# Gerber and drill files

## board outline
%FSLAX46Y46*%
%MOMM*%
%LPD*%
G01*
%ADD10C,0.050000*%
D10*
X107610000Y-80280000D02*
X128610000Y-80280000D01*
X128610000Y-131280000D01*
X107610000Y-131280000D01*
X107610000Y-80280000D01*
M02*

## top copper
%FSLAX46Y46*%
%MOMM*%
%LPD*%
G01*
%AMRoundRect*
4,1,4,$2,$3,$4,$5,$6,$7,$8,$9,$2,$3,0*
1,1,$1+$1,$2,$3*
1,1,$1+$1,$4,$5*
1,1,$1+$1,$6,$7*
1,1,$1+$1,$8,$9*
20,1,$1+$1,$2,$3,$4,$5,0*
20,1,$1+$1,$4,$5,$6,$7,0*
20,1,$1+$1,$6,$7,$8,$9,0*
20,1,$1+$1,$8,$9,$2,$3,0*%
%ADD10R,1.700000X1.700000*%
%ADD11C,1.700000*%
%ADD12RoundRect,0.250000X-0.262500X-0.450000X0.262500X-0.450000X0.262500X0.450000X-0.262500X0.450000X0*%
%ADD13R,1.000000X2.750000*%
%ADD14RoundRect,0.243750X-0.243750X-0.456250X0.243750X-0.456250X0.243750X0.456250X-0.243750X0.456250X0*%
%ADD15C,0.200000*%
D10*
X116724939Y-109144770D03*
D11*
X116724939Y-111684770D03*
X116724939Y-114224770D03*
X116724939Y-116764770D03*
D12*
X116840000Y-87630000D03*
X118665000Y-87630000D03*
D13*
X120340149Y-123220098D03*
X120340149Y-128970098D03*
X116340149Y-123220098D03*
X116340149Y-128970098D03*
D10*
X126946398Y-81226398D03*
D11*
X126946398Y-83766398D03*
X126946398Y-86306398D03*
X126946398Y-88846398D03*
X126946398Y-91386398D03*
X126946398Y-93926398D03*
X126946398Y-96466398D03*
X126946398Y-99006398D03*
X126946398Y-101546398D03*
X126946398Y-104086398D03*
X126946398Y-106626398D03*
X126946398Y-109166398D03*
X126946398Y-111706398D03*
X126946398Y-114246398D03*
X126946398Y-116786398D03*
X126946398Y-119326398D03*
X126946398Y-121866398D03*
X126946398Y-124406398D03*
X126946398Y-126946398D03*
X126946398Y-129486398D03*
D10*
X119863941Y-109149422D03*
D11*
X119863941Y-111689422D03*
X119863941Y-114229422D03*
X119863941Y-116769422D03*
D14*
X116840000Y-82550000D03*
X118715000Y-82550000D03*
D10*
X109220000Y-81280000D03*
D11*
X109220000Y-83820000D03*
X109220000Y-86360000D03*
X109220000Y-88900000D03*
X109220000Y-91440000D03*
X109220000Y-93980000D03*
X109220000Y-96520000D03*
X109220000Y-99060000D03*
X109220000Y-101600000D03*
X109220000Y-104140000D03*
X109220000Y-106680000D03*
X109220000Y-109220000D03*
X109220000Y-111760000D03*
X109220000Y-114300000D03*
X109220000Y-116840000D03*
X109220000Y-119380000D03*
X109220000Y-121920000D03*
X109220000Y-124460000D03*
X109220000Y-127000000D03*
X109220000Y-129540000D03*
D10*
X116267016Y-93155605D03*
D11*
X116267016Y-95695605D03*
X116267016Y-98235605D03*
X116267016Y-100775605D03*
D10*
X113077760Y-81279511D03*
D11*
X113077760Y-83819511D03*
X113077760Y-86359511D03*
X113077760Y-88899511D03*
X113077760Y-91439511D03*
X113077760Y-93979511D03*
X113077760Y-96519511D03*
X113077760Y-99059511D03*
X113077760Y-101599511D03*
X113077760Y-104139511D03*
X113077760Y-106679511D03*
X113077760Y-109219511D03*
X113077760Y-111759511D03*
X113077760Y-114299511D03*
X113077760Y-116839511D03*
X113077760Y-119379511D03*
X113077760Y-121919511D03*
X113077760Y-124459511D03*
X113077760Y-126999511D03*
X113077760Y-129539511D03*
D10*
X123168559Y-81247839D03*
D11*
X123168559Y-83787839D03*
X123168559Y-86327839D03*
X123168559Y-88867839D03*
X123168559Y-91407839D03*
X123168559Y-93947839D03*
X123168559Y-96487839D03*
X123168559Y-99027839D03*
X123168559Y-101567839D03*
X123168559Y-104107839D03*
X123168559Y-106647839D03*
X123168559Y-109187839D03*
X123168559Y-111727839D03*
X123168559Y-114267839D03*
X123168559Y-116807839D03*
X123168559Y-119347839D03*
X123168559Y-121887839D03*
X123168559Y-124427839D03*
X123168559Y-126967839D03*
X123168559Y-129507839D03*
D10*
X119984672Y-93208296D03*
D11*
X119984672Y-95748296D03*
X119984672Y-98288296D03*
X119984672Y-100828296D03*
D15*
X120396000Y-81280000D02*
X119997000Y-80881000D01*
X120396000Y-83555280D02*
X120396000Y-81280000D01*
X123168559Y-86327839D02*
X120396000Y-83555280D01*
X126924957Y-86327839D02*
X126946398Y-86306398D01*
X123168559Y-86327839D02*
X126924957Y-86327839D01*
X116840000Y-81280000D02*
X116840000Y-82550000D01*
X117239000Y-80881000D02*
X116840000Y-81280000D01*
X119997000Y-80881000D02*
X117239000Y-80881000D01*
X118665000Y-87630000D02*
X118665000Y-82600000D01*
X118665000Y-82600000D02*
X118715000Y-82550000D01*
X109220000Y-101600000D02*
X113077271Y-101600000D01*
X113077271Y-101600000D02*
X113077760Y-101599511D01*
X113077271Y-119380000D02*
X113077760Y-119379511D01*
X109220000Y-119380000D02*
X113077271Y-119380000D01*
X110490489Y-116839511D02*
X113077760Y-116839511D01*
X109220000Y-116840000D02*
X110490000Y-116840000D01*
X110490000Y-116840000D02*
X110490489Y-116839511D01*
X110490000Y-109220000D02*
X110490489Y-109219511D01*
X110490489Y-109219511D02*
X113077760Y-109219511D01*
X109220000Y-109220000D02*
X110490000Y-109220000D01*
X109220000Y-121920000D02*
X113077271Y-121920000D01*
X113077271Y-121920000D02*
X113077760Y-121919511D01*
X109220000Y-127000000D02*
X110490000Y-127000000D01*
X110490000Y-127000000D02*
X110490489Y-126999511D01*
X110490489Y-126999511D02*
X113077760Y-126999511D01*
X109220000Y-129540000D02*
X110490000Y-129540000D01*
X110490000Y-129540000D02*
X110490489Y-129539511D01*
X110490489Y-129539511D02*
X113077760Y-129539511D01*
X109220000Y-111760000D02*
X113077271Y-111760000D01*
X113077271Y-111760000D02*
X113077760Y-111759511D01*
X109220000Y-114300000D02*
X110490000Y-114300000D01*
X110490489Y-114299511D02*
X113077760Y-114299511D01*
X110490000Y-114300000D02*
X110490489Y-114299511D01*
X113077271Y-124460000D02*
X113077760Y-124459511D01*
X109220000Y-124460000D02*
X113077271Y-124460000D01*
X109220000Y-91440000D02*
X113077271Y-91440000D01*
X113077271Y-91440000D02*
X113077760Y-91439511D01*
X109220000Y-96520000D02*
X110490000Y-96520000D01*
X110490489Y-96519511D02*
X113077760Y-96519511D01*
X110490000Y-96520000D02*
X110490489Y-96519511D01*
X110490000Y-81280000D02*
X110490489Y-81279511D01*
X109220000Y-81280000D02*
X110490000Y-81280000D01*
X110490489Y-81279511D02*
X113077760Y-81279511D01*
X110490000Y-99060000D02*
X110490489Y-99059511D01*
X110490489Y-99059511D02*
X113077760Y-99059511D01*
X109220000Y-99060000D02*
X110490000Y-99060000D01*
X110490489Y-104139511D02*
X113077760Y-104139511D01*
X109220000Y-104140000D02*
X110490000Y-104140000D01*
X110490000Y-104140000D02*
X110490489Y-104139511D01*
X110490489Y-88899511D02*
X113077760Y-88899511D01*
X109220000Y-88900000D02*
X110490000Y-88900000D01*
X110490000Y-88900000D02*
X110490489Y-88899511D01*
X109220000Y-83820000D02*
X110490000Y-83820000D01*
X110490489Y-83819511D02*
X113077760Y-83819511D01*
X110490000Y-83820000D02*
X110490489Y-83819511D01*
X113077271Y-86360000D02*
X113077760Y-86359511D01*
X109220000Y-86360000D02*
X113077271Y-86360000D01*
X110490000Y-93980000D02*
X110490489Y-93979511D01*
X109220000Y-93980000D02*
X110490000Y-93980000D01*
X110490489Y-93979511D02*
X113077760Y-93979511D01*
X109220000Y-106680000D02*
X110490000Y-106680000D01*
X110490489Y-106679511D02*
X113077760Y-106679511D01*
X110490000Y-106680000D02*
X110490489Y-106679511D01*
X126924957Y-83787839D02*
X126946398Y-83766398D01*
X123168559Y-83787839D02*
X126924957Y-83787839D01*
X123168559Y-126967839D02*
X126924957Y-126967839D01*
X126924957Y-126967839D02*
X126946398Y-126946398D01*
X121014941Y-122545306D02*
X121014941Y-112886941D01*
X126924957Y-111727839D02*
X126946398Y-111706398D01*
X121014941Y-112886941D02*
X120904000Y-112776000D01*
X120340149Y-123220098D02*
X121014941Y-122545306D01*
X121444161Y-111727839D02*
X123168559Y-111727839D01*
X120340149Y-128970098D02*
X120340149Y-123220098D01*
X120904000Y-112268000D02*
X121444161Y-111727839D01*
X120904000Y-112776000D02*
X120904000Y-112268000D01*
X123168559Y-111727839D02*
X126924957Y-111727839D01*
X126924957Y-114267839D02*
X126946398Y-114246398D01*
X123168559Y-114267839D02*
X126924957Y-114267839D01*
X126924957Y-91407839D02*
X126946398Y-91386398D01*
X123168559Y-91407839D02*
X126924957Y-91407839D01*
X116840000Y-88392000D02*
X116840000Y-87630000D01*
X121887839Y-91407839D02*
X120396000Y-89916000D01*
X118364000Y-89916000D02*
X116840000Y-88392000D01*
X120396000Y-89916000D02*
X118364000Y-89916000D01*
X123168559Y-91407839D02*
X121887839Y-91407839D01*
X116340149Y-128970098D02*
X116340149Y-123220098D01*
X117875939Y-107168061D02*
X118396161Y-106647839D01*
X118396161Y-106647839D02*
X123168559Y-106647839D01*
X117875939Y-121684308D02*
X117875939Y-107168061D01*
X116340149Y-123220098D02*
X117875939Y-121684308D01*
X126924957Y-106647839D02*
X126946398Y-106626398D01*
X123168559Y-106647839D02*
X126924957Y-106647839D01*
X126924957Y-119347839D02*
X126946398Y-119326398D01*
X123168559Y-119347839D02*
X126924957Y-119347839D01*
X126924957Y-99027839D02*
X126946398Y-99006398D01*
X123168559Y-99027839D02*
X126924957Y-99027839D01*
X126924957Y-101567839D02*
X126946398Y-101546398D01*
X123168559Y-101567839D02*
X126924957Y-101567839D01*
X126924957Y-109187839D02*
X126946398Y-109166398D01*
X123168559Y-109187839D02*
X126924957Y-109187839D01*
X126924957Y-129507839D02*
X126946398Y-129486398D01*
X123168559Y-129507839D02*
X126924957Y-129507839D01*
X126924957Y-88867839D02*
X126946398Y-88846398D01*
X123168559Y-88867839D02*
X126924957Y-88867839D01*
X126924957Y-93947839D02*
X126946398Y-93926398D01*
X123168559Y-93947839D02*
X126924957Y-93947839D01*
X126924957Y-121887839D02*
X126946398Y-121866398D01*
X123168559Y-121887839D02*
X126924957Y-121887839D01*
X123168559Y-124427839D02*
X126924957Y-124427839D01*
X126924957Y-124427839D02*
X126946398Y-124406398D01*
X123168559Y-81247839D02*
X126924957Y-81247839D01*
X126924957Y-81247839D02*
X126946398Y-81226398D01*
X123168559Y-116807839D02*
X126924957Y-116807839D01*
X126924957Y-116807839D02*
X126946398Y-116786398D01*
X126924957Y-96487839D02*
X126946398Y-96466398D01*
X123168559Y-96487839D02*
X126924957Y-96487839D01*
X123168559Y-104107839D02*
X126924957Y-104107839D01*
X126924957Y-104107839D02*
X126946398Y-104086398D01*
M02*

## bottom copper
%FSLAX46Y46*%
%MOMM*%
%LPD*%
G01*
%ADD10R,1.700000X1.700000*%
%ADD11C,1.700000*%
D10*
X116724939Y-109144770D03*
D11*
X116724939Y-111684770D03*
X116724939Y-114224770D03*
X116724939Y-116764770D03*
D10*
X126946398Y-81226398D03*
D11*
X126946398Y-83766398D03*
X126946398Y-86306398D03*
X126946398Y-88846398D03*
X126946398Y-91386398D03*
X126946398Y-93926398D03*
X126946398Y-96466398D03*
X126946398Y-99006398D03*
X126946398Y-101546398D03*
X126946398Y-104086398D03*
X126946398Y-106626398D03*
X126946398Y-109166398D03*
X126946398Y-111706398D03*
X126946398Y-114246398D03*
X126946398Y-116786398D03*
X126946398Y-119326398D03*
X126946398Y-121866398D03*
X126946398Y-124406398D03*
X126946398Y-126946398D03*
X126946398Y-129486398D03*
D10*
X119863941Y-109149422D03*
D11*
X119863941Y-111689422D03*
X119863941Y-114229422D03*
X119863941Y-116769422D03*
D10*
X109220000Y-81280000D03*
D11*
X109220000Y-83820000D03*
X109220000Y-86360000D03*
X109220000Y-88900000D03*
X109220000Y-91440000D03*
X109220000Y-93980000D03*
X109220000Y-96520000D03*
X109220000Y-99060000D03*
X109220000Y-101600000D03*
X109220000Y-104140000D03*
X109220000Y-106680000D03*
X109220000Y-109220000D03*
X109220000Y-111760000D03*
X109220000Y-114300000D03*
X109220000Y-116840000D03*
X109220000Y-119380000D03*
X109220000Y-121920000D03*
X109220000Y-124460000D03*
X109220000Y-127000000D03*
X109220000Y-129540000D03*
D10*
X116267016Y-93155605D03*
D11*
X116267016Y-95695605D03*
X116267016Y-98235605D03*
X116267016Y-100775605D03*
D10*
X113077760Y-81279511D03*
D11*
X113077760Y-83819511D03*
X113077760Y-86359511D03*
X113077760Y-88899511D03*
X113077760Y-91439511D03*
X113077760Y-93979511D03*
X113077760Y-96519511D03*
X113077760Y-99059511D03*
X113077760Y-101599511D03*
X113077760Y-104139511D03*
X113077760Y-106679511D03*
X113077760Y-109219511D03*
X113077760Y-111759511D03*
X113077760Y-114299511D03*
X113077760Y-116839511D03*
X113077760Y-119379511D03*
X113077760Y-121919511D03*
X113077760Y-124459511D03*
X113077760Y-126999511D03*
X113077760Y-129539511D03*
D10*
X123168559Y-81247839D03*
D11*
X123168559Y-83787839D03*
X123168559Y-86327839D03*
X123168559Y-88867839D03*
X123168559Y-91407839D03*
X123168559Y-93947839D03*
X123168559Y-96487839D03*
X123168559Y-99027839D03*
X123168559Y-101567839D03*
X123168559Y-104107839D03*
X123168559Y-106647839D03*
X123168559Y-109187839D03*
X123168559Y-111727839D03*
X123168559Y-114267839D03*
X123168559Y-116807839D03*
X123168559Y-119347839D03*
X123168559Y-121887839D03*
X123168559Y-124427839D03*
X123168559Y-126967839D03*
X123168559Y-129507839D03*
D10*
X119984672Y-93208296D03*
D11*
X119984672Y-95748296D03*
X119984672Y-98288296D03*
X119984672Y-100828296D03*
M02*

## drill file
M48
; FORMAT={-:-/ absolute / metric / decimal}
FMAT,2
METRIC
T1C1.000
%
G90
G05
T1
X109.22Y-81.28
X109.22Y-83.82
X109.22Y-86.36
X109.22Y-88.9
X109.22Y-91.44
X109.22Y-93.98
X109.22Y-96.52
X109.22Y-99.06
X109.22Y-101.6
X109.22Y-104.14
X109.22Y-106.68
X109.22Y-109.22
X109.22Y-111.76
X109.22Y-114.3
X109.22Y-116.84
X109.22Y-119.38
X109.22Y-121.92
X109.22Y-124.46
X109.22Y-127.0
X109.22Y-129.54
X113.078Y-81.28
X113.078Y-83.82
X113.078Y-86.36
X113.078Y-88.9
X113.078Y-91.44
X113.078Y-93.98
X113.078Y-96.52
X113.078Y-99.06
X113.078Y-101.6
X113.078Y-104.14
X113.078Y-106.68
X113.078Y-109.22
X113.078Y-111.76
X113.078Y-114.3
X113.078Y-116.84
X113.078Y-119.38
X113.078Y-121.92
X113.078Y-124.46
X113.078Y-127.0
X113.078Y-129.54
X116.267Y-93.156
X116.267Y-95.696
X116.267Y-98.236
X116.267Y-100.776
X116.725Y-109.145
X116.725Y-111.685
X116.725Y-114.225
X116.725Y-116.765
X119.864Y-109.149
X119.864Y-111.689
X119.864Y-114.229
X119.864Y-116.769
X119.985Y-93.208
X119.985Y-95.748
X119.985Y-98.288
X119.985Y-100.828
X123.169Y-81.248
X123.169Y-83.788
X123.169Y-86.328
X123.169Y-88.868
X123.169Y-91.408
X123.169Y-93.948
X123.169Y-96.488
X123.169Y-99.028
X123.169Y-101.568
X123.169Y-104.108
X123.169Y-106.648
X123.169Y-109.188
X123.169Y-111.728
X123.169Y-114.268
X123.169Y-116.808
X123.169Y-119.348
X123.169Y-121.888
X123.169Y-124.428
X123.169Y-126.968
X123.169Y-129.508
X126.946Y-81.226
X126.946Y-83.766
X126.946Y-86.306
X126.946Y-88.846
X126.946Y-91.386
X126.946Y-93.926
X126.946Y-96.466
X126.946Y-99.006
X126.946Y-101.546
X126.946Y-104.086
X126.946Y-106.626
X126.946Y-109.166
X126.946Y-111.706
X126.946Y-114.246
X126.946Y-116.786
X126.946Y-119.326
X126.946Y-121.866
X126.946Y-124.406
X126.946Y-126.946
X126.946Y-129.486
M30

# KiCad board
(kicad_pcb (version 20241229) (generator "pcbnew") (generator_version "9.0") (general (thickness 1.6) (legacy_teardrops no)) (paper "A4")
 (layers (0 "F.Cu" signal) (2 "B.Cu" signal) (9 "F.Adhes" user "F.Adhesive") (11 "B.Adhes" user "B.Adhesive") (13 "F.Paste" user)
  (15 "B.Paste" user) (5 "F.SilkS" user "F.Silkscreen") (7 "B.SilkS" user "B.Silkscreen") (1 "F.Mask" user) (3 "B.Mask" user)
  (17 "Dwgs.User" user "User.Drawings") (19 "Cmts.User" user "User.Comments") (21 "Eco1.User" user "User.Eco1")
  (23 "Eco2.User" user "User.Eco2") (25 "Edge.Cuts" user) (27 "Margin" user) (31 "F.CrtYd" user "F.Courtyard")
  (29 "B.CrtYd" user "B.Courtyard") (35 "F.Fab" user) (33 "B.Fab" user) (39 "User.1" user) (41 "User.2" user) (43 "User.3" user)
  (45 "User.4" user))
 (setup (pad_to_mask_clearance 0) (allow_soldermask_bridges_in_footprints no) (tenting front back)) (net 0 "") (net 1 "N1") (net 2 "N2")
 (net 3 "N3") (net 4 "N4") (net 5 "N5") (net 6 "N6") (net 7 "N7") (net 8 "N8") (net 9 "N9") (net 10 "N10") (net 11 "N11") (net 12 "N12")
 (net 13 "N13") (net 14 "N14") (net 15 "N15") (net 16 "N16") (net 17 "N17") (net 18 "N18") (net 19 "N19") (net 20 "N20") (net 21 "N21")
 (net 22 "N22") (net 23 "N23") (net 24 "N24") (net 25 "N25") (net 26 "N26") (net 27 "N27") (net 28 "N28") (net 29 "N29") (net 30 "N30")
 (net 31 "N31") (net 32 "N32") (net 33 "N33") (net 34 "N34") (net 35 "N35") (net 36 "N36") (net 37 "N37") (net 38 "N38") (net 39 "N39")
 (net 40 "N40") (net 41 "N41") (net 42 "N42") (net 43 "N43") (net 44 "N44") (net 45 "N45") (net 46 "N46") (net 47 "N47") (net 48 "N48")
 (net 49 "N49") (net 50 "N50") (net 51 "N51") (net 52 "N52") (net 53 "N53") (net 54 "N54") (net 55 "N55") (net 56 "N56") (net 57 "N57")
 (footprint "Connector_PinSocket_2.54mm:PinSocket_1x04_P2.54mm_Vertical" (layer "F.Cu") (at 116.724939 109.14477)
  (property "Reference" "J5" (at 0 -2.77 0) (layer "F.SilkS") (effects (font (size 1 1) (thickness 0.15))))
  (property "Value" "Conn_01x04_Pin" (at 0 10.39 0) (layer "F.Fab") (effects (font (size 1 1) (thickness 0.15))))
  (pad "1" thru_hole rect (at 0 0) (size 1.7 1.7) (drill 1) (layers "*.Cu" "*.Mask") (remove_unused_layers no) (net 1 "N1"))
  (pad "2" thru_hole circle (at 0 2.54) (size 1.7 1.7) (drill 1) (layers "*.Cu" "*.Mask") (remove_unused_layers no) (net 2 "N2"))
  (pad "3" thru_hole circle (at 0 5.08) (size 1.7 1.7) (drill 1) (layers "*.Cu" "*.Mask") (remove_unused_layers no) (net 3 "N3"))
  (pad "4" thru_hole circle (at 0 7.62) (size 1.7 1.7) (drill 1) (layers "*.Cu" "*.Mask") (remove_unused_layers no) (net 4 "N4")))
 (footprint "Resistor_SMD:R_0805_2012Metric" (layer "F.Cu") (at 117.7525 87.63)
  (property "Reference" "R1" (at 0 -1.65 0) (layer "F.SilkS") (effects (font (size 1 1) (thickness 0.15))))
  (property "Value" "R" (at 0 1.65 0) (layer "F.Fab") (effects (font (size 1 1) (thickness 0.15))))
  (pad "1" smd roundrect (at -0.9125 0) (size 1.025 1.4) (layers "F.Cu" "F.Mask" "F.Paste") (roundrect_rratio 0.243902) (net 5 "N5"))
  (pad "2" smd roundrect (at 0.9125 0) (size 1.025 1.4) (layers "F.Cu" "F.Mask" "F.Paste") (roundrect_rratio 0.243902) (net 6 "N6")))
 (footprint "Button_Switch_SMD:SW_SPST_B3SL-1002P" (layer "F.Cu") (at 118.340149 126.095098 -90)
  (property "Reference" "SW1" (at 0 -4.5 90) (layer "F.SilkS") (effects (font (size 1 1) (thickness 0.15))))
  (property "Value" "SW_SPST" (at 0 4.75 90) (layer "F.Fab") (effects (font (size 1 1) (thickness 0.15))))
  (pad "1" smd rect (at -2.875 -2 270) (size 2.75 1) (layers "F.Cu" "F.Mask" "F.Paste") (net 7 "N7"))
  (pad "1" smd rect (at 2.875 -2 270) (size 2.75 1) (layers "F.Cu" "F.Mask" "F.Paste") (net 7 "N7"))
  (pad "2" smd rect (at -2.875 2 270) (size 2.75 1) (layers "F.Cu" "F.Mask" "F.Paste") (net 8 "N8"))
  (pad "2" smd rect (at 2.875 2 270) (size 2.75 1) (layers "F.Cu" "F.Mask" "F.Paste") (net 8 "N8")))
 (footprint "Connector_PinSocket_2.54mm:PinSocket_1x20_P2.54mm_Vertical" (layer "F.Cu") (at 126.946398 81.226398)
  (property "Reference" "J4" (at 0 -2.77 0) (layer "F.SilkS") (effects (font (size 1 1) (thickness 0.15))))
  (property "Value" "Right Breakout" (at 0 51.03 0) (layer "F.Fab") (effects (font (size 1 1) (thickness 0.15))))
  (pad "1" thru_hole rect (at 0 0) (size 1.7 1.7) (drill 1) (layers "*.Cu" "*.Mask") (remove_unused_layers no) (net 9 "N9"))
  (pad "2" thru_hole circle (at 0 2.54) (size 1.7 1.7) (drill 1) (layers "*.Cu" "*.Mask") (remove_unused_layers no) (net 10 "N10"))
  (pad "3" thru_hole circle (at 0 5.08) (size 1.7 1.7) (drill 1) (layers "*.Cu" "*.Mask") (remove_unused_layers no) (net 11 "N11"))
  (pad "4" thru_hole circle (at 0 7.62) (size 1.7 1.7) (drill 1) (layers "*.Cu" "*.Mask") (remove_unused_layers no) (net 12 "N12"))
  (pad "5" thru_hole circle (at 0 10.16) (size 1.7 1.7) (drill 1) (layers "*.Cu" "*.Mask") (remove_unused_layers no) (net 5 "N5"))
  (pad "6" thru_hole circle (at 0 12.7) (size 1.7 1.7) (drill 1) (layers "*.Cu" "*.Mask") (remove_unused_layers no) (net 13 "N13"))
  (pad "7" thru_hole circle (at 0 15.24) (size 1.7 1.7) (drill 1) (layers "*.Cu" "*.Mask") (remove_unused_layers no) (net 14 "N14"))
  (pad "8" thru_hole circle (at 0 17.78) (size 1.7 1.7) (drill 1) (layers "*.Cu" "*.Mask") (remove_unused_layers no) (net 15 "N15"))
  (pad "9" thru_hole circle (at 0 20.32) (size 1.7 1.7) (drill 1) (layers "*.Cu" "*.Mask") (remove_unused_layers no) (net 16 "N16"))
  (pad "10" thru_hole circle (at 0 22.86) (size 1.7 1.7) (drill 1) (layers "*.Cu" "*.Mask") (remove_unused_layers no) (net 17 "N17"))
  (pad "11" thru_hole circle (at 0 25.4) (size 1.7 1.7) (drill 1) (layers "*.Cu" "*.Mask") (remove_unused_layers no) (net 8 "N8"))
  (pad "12" thru_hole circle (at 0 27.94) (size 1.7 1.7) (drill 1) (layers "*.Cu" "*.Mask") (remove_unused_layers no) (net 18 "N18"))
  (pad "13" thru_hole circle (at 0 30.48) (size 1.7 1.7) (drill 1) (layers "*.Cu" "*.Mask") (remove_unused_layers no) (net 7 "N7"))
  (pad "14" thru_hole circle (at 0 33.02) (size 1.7 1.7) (drill 1) (layers "*.Cu" "*.Mask") (remove_unused_layers no) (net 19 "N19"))
  (pad "15" thru_hole circle (at 0 35.56) (size 1.7 1.7) (drill 1) (layers "*.Cu" "*.Mask") (remove_unused_layers no) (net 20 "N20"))
  (pad "16" thru_hole circle (at 0 38.1) (size 1.7 1.7) (drill 1) (layers "*.Cu" "*.Mask") (remove_unused_layers no) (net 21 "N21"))
  (pad "17" thru_hole circle (at 0 40.64) (size 1.7 1.7) (drill 1) (layers "*.Cu" "*.Mask") (remove_unused_layers no) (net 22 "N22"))
  (pad "18" thru_hole circle (at 0 43.18) (size 1.7 1.7) (drill 1) (layers "*.Cu" "*.Mask") (remove_unused_layers no) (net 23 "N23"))
  (pad "19" thru_hole circle (at 0 45.72) (size 1.7 1.7) (drill 1) (layers "*.Cu" "*.Mask") (remove_unused_layers no) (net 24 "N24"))
  (pad "20" thru_hole circle (at 0 48.26) (size 1.7 1.7) (drill 1) (layers "*.Cu" "*.Mask") (remove_unused_layers no) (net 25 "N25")))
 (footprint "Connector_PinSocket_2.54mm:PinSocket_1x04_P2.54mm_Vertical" (layer "F.Cu") (at 119.863941 109.149422)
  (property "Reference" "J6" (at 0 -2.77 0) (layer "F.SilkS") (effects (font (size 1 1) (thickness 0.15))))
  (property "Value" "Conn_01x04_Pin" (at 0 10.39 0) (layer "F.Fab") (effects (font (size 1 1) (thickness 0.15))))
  (pad "1" thru_hole rect (at 0 0) (size 1.7 1.7) (drill 1) (layers "*.Cu" "*.Mask") (remove_unused_layers no) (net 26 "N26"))
  (pad "2" thru_hole circle (at 0 2.54) (size 1.7 1.7) (drill 1) (layers "*.Cu" "*.Mask") (remove_unused_layers no) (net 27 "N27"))
  (pad "3" thru_hole circle (at 0 5.08) (size 1.7 1.7) (drill 1) (layers "*.Cu" "*.Mask") (remove_unused_layers no) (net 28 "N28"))
  (pad "4" thru_hole circle (at 0 7.62) (size 1.7 1.7) (drill 1) (layers "*.Cu" "*.Mask") (remove_unused_layers no) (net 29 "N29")))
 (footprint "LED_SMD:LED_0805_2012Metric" (layer "F.Cu") (at 117.7775 82.55)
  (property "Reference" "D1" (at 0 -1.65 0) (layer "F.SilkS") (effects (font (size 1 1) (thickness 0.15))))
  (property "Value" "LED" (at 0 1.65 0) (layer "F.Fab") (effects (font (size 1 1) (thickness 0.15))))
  (pad "1" smd roundrect (at -0.9375 0) (size 0.975 1.4) (layers "F.Cu" "F.Mask" "F.Paste") (roundrect_rratio 0.25) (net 11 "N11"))
  (pad "2" smd roundrect (at 0.9375 0) (size 0.975 1.4) (layers "F.Cu" "F.Mask" "F.Paste") (roundrect_rratio 0.25) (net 6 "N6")))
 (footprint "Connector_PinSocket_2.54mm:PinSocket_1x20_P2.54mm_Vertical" (layer "F.Cu") (at 109.22 81.28)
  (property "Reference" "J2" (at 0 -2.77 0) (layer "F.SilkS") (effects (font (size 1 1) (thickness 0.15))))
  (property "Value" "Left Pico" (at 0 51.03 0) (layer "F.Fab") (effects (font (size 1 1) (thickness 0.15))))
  (pad "1" thru_hole rect (at 0 0) (size 1.7 1.7) (drill 1) (layers "*.Cu" "*.Mask") (remove_unused_layers no) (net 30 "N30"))
  (pad "2" thru_hole circle (at 0 2.54) (size 1.7 1.7) (drill 1) (layers "*.Cu" "*.Mask") (remove_unused_layers no) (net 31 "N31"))
  (pad "3" thru_hole circle (at 0 5.08) (size 1.7 1.7) (drill 1) (layers "*.Cu" "*.Mask") (remove_unused_layers no) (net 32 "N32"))
  (pad "4" thru_hole circle (at 0 7.62) (size 1.7 1.7) (drill 1) (layers "*.Cu" "*.Mask") (remove_unused_layers no) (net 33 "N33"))
  (pad "5" thru_hole circle (at 0 10.16) (size 1.7 1.7) (drill 1) (layers "*.Cu" "*.Mask") (remove_unused_layers no) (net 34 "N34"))
  (pad "6" thru_hole circle (at 0 12.7) (size 1.7 1.7) (drill 1) (layers "*.Cu" "*.Mask") (remove_unused_layers no) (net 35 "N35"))
  (pad "7" thru_hole circle (at 0 15.24) (size 1.7 1.7) (drill 1) (layers "*.Cu" "*.Mask") (remove_unused_layers no) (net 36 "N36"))
  (pad "8" thru_hole circle (at 0 17.78) (size 1.7 1.7) (drill 1) (layers "*.Cu" "*.Mask") (remove_unused_layers no) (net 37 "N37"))
  (pad "9" thru_hole circle (at 0 20.32) (size 1.7 1.7) (drill 1) (layers "*.Cu" "*.Mask") (remove_unused_layers no) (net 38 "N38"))
  (pad "10" thru_hole circle (at 0 22.86) (size 1.7 1.7) (drill 1) (layers "*.Cu" "*.Mask") (remove_unused_layers no) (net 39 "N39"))
  (pad "11" thru_hole circle (at 0 25.4) (size 1.7 1.7) (drill 1) (layers "*.Cu" "*.Mask") (remove_unused_layers no) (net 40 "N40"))
  (pad "12" thru_hole circle (at 0 27.94) (size 1.7 1.7) (drill 1) (layers "*.Cu" "*.Mask") (remove_unused_layers no) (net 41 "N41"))
  (pad "13" thru_hole circle (at 0 30.48) (size 1.7 1.7) (drill 1) (layers "*.Cu" "*.Mask") (remove_unused_layers no) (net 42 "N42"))
  (pad "14" thru_hole circle (at 0 33.02) (size 1.7 1.7) (drill 1) (layers "*.Cu" "*.Mask") (remove_unused_layers no) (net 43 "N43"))
  (pad "15" thru_hole circle (at 0 35.56) (size 1.7 1.7) (drill 1) (layers "*.Cu" "*.Mask") (remove_unused_layers no) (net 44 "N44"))
  (pad "16" thru_hole circle (at 0 38.1) (size 1.7 1.7) (drill 1) (layers "*.Cu" "*.Mask") (remove_unused_layers no) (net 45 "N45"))
  (pad "17" thru_hole circle (at 0 40.64) (size 1.7 1.7) (drill 1) (layers "*.Cu" "*.Mask") (remove_unused_layers no) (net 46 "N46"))
  (pad "18" thru_hole circle (at 0 43.18) (size 1.7 1.7) (drill 1) (layers "*.Cu" "*.Mask") (remove_unused_layers no) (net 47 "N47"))
  (pad "19" thru_hole circle (at 0 45.72) (size 1.7 1.7) (drill 1) (layers "*.Cu" "*.Mask") (remove_unused_layers no) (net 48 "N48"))
  (pad "20" thru_hole circle (at 0 48.26) (size 1.7 1.7) (drill 1) (layers "*.Cu" "*.Mask") (remove_unused_layers no) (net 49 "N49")))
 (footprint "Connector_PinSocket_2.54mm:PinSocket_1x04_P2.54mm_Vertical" (layer "F.Cu") (at 116.267016 93.155605)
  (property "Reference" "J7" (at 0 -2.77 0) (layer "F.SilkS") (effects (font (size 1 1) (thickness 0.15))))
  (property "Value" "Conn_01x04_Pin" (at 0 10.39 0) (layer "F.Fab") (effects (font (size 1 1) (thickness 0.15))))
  (pad "1" thru_hole rect (at 0 0) (size 1.7 1.7) (drill 1) (layers "*.Cu" "*.Mask") (remove_unused_layers no) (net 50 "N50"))
  (pad "2" thru_hole circle (at 0 2.54) (size 1.7 1.7) (drill 1) (layers "*.Cu" "*.Mask") (remove_unused_layers no) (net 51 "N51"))
  (pad "3" thru_hole circle (at 0 5.08) (size 1.7 1.7) (drill 1) (layers "*.Cu" "*.Mask") (remove_unused_layers no) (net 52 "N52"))
  (pad "4" thru_hole circle (at 0 7.62) (size 1.7 1.7) (drill 1) (layers "*.Cu" "*.Mask") (remove_unused_layers no) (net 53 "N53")))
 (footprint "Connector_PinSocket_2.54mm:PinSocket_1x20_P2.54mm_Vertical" (layer "F.Cu") (at 113.07776 81.279511)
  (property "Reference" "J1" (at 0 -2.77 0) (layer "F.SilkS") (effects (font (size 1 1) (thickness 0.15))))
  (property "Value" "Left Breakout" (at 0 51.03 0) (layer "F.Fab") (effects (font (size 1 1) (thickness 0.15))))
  (pad "1" thru_hole rect (at 0 0) (size 1.7 1.7) (drill 1) (layers "*.Cu" "*.Mask") (remove_unused_layers no) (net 30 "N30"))
  (pad "2" thru_hole circle (at 0 2.54) (size 1.7 1.7) (drill 1) (layers "*.Cu" "*.Mask") (remove_unused_layers no) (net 31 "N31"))
  (pad "3" thru_hole circle (at 0 5.08) (size 1.7 1.7) (drill 1) (layers "*.Cu" "*.Mask") (remove_unused_layers no) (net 32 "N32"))
  (pad "4" thru_hole circle (at 0 7.62) (size 1.7 1.7) (drill 1) (layers "*.Cu" "*.Mask") (remove_unused_layers no) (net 33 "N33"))
  (pad "5" thru_hole circle (at 0 10.16) (size 1.7 1.7) (drill 1) (layers "*.Cu" "*.Mask") (remove_unused_layers no) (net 34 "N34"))
  (pad "6" thru_hole circle (at 0 12.7) (size 1.7 1.7) (drill 1) (layers "*.Cu" "*.Mask") (remove_unused_layers no) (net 35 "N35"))
  (pad "7" thru_hole circle (at 0 15.24) (size 1.7 1.7) (drill 1) (layers "*.Cu" "*.Mask") (remove_unused_layers no) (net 36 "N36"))
  (pad "8" thru_hole circle (at 0 17.78) (size 1.7 1.7) (drill 1) (layers "*.Cu" "*.Mask") (remove_unused_layers no) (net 37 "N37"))
  (pad "9" thru_hole circle (at 0 20.32) (size 1.7 1.7) (drill 1) (layers "*.Cu" "*.Mask") (remove_unused_layers no) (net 38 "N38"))
  (pad "10" thru_hole circle (at 0 22.86) (size 1.7 1.7) (drill 1) (layers "*.Cu" "*.Mask") (remove_unused_layers no) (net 39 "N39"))
  (pad "11" thru_hole circle (at 0 25.4) (size 1.7 1.7) (drill 1) (layers "*.Cu" "*.Mask") (remove_unused_layers no) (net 40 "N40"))
  (pad "12" thru_hole circle (at 0 27.94) (size 1.7 1.7) (drill 1) (layers "*.Cu" "*.Mask") (remove_unused_layers no) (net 41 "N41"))
  (pad "13" thru_hole circle (at 0 30.48) (size 1.7 1.7) (drill 1) (layers "*.Cu" "*.Mask") (remove_unused_layers no) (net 42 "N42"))
  (pad "14" thru_hole circle (at 0 33.02) (size 1.7 1.7) (drill 1) (layers "*.Cu" "*.Mask") (remove_unused_layers no) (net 43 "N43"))
  (pad "15" thru_hole circle (at 0 35.56) (size 1.7 1.7) (drill 1) (layers "*.Cu" "*.Mask") (remove_unused_layers no) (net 44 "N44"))
  (pad "16" thru_hole circle (at 0 38.1) (size 1.7 1.7) (drill 1) (layers "*.Cu" "*.Mask") (remove_unused_layers no) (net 45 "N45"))
  (pad "17" thru_hole circle (at 0 40.64) (size 1.7 1.7) (drill 1) (layers "*.Cu" "*.Mask") (remove_unused_layers no) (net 46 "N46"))
  (pad "18" thru_hole circle (at 0 43.18) (size 1.7 1.7) (drill 1) (layers "*.Cu" "*.Mask") (remove_unused_layers no) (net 47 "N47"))
  (pad "19" thru_hole circle (at 0 45.72) (size 1.7 1.7) (drill 1) (layers "*.Cu" "*.Mask") (remove_unused_layers no) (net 48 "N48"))
  (pad "20" thru_hole circle (at 0 48.26) (size 1.7 1.7) (drill 1) (layers "*.Cu" "*.Mask") (remove_unused_layers no) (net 49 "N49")))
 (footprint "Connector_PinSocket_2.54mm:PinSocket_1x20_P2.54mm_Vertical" (layer "F.Cu") (at 123.168559 81.247839)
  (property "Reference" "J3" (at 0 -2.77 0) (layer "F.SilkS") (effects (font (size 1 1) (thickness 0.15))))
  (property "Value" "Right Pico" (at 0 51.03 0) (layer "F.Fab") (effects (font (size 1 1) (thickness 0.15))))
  (pad "1" thru_hole rect (at 0 0) (size 1.7 1.7) (drill 1) (layers "*.Cu" "*.Mask") (remove_unused_layers no) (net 9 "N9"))
  (pad "2" thru_hole circle (at 0 2.54) (size 1.7 1.7) (drill 1) (layers "*.Cu" "*.Mask") (remove_unused_layers no) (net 10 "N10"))
  (pad "3" thru_hole circle (at 0 5.08) (size 1.7 1.7) (drill 1) (layers "*.Cu" "*.Mask") (remove_unused_layers no) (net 11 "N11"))
  (pad "4" thru_hole circle (at 0 7.62) (size 1.7 1.7) (drill 1) (layers "*.Cu" "*.Mask") (remove_unused_layers no) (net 12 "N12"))
  (pad "5" thru_hole circle (at 0 10.16) (size 1.7 1.7) (drill 1) (layers "*.Cu" "*.Mask") (remove_unused_layers no) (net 5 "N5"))
  (pad "6" thru_hole circle (at 0 12.7) (size 1.7 1.7) (drill 1) (layers "*.Cu" "*.Mask") (remove_unused_layers no) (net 13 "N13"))
  (pad "7" thru_hole circle (at 0 15.24) (size 1.7 1.7) (drill 1) (layers "*.Cu" "*.Mask") (remove_unused_layers no) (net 14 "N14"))
  (pad "8" thru_hole circle (at 0 17.78) (size 1.7 1.7) (drill 1) (layers "*.Cu" "*.Mask") (remove_unused_layers no) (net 15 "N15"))
  (pad "9" thru_hole circle (at 0 20.32) (size 1.7 1.7) (drill 1) (layers "*.Cu" "*.Mask") (remove_unused_layers no) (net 16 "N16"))
  (pad "10" thru_hole circle (at 0 22.86) (size 1.7 1.7) (drill 1) (layers "*.Cu" "*.Mask") (remove_unused_layers no) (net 17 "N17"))
  (pad "11" thru_hole circle (at 0 25.4) (size 1.7 1.7) (drill 1) (layers "*.Cu" "*.Mask") (remove_unused_layers no) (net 8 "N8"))
  (pad "12" thru_hole circle (at 0 27.94) (size 1.7 1.7) (drill 1) (layers "*.Cu" "*.Mask") (remove_unused_layers no) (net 18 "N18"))
  (pad "13" thru_hole circle (at 0 30.48) (size 1.7 1.7) (drill 1) (layers "*.Cu" "*.Mask") (remove_unused_layers no) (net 7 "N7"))
  (pad "14" thru_hole circle (at 0 33.02) (size 1.7 1.7) (drill 1) (layers "*.Cu" "*.Mask") (remove_unused_layers no) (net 19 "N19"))
  (pad "15" thru_hole circle (at 0 35.56) (size 1.7 1.7) (drill 1) (layers "*.Cu" "*.Mask") (remove_unused_layers no) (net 20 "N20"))
  (pad "16" thru_hole circle (at 0 38.1) (size 1.7 1.7) (drill 1) (layers "*.Cu" "*.Mask") (remove_unused_layers no) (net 21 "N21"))
  (pad "17" thru_hole circle (at 0 40.64) (size 1.7 1.7) (drill 1) (layers "*.Cu" "*.Mask") (remove_unused_layers no) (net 22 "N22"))
  (pad "18" thru_hole circle (at 0 43.18) (size 1.7 1.7) (drill 1) (layers "*.Cu" "*.Mask") (remove_unused_layers no) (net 23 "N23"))
  (pad "19" thru_hole circle (at 0 45.72) (size 1.7 1.7) (drill 1) (layers "*.Cu" "*.Mask") (remove_unused_layers no) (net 24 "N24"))
  (pad "20" thru_hole circle (at 0 48.26) (size 1.7 1.7) (drill 1) (layers "*.Cu" "*.Mask") (remove_unused_layers no) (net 25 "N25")))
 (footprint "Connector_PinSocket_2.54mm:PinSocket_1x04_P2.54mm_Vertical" (layer "F.Cu") (at 119.984672 93.208296)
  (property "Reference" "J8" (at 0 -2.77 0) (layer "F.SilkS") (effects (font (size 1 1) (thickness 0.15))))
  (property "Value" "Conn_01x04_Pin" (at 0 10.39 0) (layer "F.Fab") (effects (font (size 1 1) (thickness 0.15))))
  (pad "1" thru_hole rect (at 0 0) (size 1.7 1.7) (drill 1) (layers "*.Cu" "*.Mask") (remove_unused_layers no) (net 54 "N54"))
  (pad "2" thru_hole circle (at 0 2.54) (size 1.7 1.7) (drill 1) (layers "*.Cu" "*.Mask") (remove_unused_layers no) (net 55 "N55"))
  (pad "3" thru_hole circle (at 0 5.08) (size 1.7 1.7) (drill 1) (layers "*.Cu" "*.Mask") (remove_unused_layers no) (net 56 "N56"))
  (pad "4" thru_hole circle (at 0 7.62) (size 1.7 1.7) (drill 1) (layers "*.Cu" "*.Mask") (remove_unused_layers no) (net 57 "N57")))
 (gr_rect (start 107.61 80.28) (end 128.61 131.28) (stroke (width 0.05) (type solid)) (fill no) (layer "Edge.Cuts"))
 (segment (start 120.396 81.28) (end 119.997 80.881) (width 0.2) (layer "F.Cu") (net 11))
 (segment (start 120.396 83.55528) (end 120.396 81.28) (width 0.2) (layer "F.Cu") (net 11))
 (segment (start 123.168559 86.327839) (end 120.396 83.55528) (width 0.2) (layer "F.Cu") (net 11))
 (segment (start 126.924957 86.327839) (end 126.946398 86.306398) (width 0.2) (layer "F.Cu") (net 11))
 (segment (start 123.168559 86.327839) (end 126.924957 86.327839) (width 0.2) (layer "F.Cu") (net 11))
 (segment (start 116.84 81.28) (end 116.84 82.55) (width 0.2) (layer "F.Cu") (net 11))
 (segment (start 117.239 80.881) (end 116.84 81.28) (width 0.2) (layer "F.Cu") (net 11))
 (segment (start 119.997 80.881) (end 117.239 80.881) (width 0.2) (layer "F.Cu") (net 11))
 (segment (start 118.665 87.63) (end 118.665 82.6) (width 0.2) (layer "F.Cu") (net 6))
 (segment (start 118.665 82.6) (end 118.715 82.55) (width 0.2) (layer "F.Cu") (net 6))
 (segment (start 109.22 101.6) (end 113.077271 101.6) (width 0.2) (layer "F.Cu") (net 38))
 (segment (start 113.077271 101.6) (end 113.07776 101.599511) (width 0.2) (layer "F.Cu") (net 38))
 (segment (start 113.077271 119.38) (end 113.07776 119.379511) (width 0.2) (layer "F.Cu") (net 45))
 (segment (start 109.22 119.38) (end 113.077271 119.38) (width 0.2) (layer "F.Cu") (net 45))
 (segment (start 110.490489 116.839511) (end 113.07776 116.839511) (width 0.2) (layer "F.Cu") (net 44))
 (segment (start 109.22 116.84) (end 110.49 116.84) (width 0.2) (layer "F.Cu") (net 44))
 (segment (start 110.49 116.84) (end 110.490489 116.839511) (width 0.2) (layer "F.Cu") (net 44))
 (segment (start 110.49 109.22) (end 110.490489 109.219511) (width 0.2) (layer "F.Cu") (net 41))
 (segment (start 110.490489 109.219511) (end 113.07776 109.219511) (width 0.2) (layer "F.Cu") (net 41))
 (segment (start 109.22 109.22) (end 110.49 109.22) (width 0.2) (layer "F.Cu") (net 41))
 (segment (start 109.22 121.92) (end 113.077271 121.92) (width 0.2) (layer "F.Cu") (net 46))
 (segment (start 113.077271 121.92) (end 113.07776 121.919511) (width 0.2) (layer "F.Cu") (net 46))
 (segment (start 109.22 127) (end 110.49 127) (width 0.2) (layer "F.Cu") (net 48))
 (segment (start 110.49 127) (end 110.490489 126.999511) (width 0.2) (layer "F.Cu") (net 48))
 (segment (start 110.490489 126.999511) (end 113.07776 126.999511) (width 0.2) (layer "F.Cu") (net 48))
 (segment (start 109.22 129.54) (end 110.49 129.54) (width 0.2) (layer "F.Cu") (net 49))
 (segment (start 110.49 129.54) (end 110.490489 129.539511) (width 0.2) (layer "F.Cu") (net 49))
 (segment (start 110.490489 129.539511) (end 113.07776 129.539511) (width 0.2) (layer "F.Cu") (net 49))
 (segment (start 109.22 111.76) (end 113.077271 111.76) (width 0.2) (layer "F.Cu") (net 42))
 (segment (start 113.077271 111.76) (end 113.07776 111.759511) (width 0.2) (layer "F.Cu") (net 42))
 (segment (start 109.22 114.3) (end 110.49 114.3) (width 0.2) (layer "F.Cu") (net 43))
 (segment (start 110.490489 114.299511) (end 113.07776 114.299511) (width 0.2) (layer "F.Cu") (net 43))
 (segment (start 110.49 114.3) (end 110.490489 114.299511) (width 0.2) (layer "F.Cu") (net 43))
 (segment (start 113.077271 124.46) (end 113.07776 124.459511) (width 0.2) (layer "F.Cu") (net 47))
 (segment (start 109.22 124.46) (end 113.077271 124.46) (width 0.2) (layer "F.Cu") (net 47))
 (segment (start 109.22 91.44) (end 113.077271 91.44) (width 0.2) (layer "F.Cu") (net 34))
 (segment (start 113.077271 91.44) (end 113.07776 91.439511) (width 0.2) (layer "F.Cu") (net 34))
 (segment (start 109.22 96.52) (end 110.49 96.52) (width 0.2) (layer "F.Cu") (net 36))
 (segment (start 110.490489 96.519511) (end 113.07776 96.519511) (width 0.2) (layer "F.Cu") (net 36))
 (segment (start 110.49 96.52) (end 110.490489 96.519511) (width 0.2) (layer "F.Cu") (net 36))
 (segment (start 110.49 81.28) (end 110.490489 81.279511) (width 0.2) (layer "F.Cu") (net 30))
 (segment (start 109.22 81.28) (end 110.49 81.28) (width 0.2) (layer "F.Cu") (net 30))
 (segment (start 110.490489 81.279511) (end 113.07776 81.279511) (width 0.2) (layer "F.Cu") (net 30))
 (segment (start 110.49 99.06) (end 110.490489 99.059511) (width 0.2) (layer "F.Cu") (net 37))
 (segment (start 110.490489 99.059511) (end 113.07776 99.059511) (width 0.2) (layer "F.Cu") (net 37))
 (segment (start 109.22 99.06) (end 110.49 99.06) (width 0.2) (layer "F.Cu") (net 37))
 (segment (start 110.490489 104.139511) (end 113.07776 104.139511) (width 0.2) (layer "F.Cu") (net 39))
 (segment (start 109.22 104.14) (end 110.49 104.14) (width 0.2) (layer "F.Cu") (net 39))
 (segment (start 110.49 104.14) (end 110.490489 104.139511) (width 0.2) (layer "F.Cu") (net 39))
 (segment (start 110.490489 88.899511) (end 113.07776 88.899511) (width 0.2) (layer "F.Cu") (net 33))
 (segment (start 109.22 88.9) (end 110.49 88.9) (width 0.2) (layer "F.Cu") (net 33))
 (segment (start 110.49 88.9) (end 110.490489 88.899511) (width 0.2) (layer "F.Cu") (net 33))
 (segment (start 109.22 83.82) (end 110.49 83.82) (width 0.2) (layer "F.Cu") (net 31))
 (segment (start 110.490489 83.819511) (end 113.07776 83.819511) (width 0.2) (layer "F.Cu") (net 31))
 (segment (start 110.49 83.82) (end 110.490489 83.819511) (width 0.2) (layer "F.Cu") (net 31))
 (segment (start 113.077271 86.36) (end 113.07776 86.359511) (width 0.2) (layer "F.Cu") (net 32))
 (segment (start 109.22 86.36) (end 113.077271 86.36) (width 0.2) (layer "F.Cu") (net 32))
 (segment (start 110.49 93.98) (end 110.490489 93.979511) (width 0.2) (layer "F.Cu") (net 35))
 (segment (start 109.22 93.98) (end 110.49 93.98) (width 0.2) (layer "F.Cu") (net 35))
 (segment (start 110.490489 93.979511) (end 113.07776 93.979511) (width 0.2) (layer "F.Cu") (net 35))
 (segment (start 109.22 106.68) (end 110.49 106.68) (width 0.2) (layer "F.Cu") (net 40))
 (segment (start 110.490489 106.679511) (end 113.07776 106.679511) (width 0.2) (layer "F.Cu") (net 40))
 (segment (start 110.49 106.68) (end 110.490489 106.679511) (width 0.2) (layer "F.Cu") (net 40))
 (segment (start 126.924957 83.787839) (end 126.946398 83.766398) (width 0.2) (layer "F.Cu") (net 10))
 (segment (start 123.168559 83.787839) (end 126.924957 83.787839) (width 0.2) (layer "F.Cu") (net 10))
 (segment (start 123.168559 126.967839) (end 126.924957 126.967839) (width 0.2) (layer "F.Cu") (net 24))
 (segment (start 126.924957 126.967839) (end 126.946398 126.946398) (width 0.2) (layer "F.Cu") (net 24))
 (segment (start 121.014941 122.545306) (end 121.014941 112.886941) (width 0.2) (layer "F.Cu") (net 7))
 (segment (start 126.924957 111.727839) (end 126.946398 111.706398) (width 0.2) (layer "F.Cu") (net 7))
 (segment (start 121.014941 112.886941) (end 120.904 112.776) (width 0.2) (layer "F.Cu") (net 7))
 (segment (start 120.340149 123.220098) (end 121.014941 122.545306) (width 0.2) (layer "F.Cu") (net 7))
 (segment (start 121.444161 111.727839) (end 123.168559 111.727839) (width 0.2) (layer "F.Cu") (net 7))
 (segment (start 120.340149 128.970098) (end 120.340149 123.220098) (width 0.2) (layer "F.Cu") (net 7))
 (segment (start 120.904 112.268) (end 121.444161 111.727839) (width 0.2) (layer "F.Cu") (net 7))
 (segment (start 120.904 112.776) (end 120.904 112.268) (width 0.2) (layer "F.Cu") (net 7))
 (segment (start 123.168559 111.727839) (end 126.924957 111.727839) (width 0.2) (layer "F.Cu") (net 7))
 (segment (start 126.924957 114.267839) (end 126.946398 114.246398) (width 0.2) (layer "F.Cu") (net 19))
 (segment (start 123.168559 114.267839) (end 126.924957 114.267839) (width 0.2) (layer "F.Cu") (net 19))
 (segment (start 126.924957 91.407839) (end 126.946398 91.386398) (width 0.2) (layer "F.Cu") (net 5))
 (segment (start 123.168559 91.407839) (end 126.924957 91.407839) (width 0.2) (layer "F.Cu") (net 5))
 (segment (start 116.84 88.392) (end 116.84 87.63) (width 0.2) (layer "F.Cu") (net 5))
 (segment (start 121.887839 91.407839) (end 120.396 89.916) (width 0.2) (layer "F.Cu") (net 5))
 (segment (start 118.364 89.916) (end 116.84 88.392) (width 0.2) (layer "F.Cu") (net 5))
 (segment (start 120.396 89.916) (end 118.364 89.916) (width 0.2) (layer "F.Cu") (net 5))
 (segment (start 123.168559 91.407839) (end 121.887839 91.407839) (width 0.2) (layer "F.Cu") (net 5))
 (segment (start 116.340149 128.970098) (end 116.340149 123.220098) (width 0.2) (layer "F.Cu") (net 8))
 (segment (start 117.875939 107.168061) (end 118.396161 106.647839) (width 0.2) (layer "F.Cu") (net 8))
 (segment (start 118.396161 106.647839) (end 123.168559 106.647839) (width 0.2) (layer "F.Cu") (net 8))
 (segment (start 117.875939 121.684308) (end 117.875939 107.168061) (width 0.2) (layer "F.Cu") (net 8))
 (segment (start 116.340149 123.220098) (end 117.875939 121.684308) (width 0.2) (layer "F.Cu") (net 8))
 (segment (start 126.924957 106.647839) (end 126.946398 106.626398) (width 0.2) (layer "F.Cu") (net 8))
 (segment (start 123.168559 106.647839) (end 126.924957 106.647839) (width 0.2) (layer "F.Cu") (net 8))
 (segment (start 126.924957 119.347839) (end 126.946398 119.326398) (width 0.2) (layer "F.Cu") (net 21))
 (segment (start 123.168559 119.347839) (end 126.924957 119.347839) (width 0.2) (layer "F.Cu") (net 21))
 (segment (start 126.924957 99.027839) (end 126.946398 99.006398) (width 0.2) (layer "F.Cu") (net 15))
 (segment (start 123.168559 99.027839) (end 126.924957 99.027839) (width 0.2) (layer "F.Cu") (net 15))
 (segment (start 126.924957 101.567839) (end 126.946398 101.546398) (width 0.2) (layer "F.Cu") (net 16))
 (segment (start 123.168559 101.567839) (end 126.924957 101.567839) (width 0.2) (layer "F.Cu") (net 16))
 (segment (start 126.924957 109.187839) (end 126.946398 109.166398) (width 0.2) (layer "F.Cu") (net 18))
 (segment (start 123.168559 109.187839) (end 126.924957 109.187839) (width 0.2) (layer "F.Cu") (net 18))
 (segment (start 126.924957 129.507839) (end 126.946398 129.486398) (width 0.2) (layer "F.Cu") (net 25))
 (segment (start 123.168559 129.507839) (end 126.924957 129.507839) (width 0.2) (layer "F.Cu") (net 25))
 (segment (start 126.924957 88.867839) (end 126.946398 88.846398) (width 0.2) (layer "F.Cu") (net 12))
 (segment (start 123.168559 88.867839) (end 126.924957 88.867839) (width 0.2) (layer "F.Cu") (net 12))
 (segment (start 126.924957 93.947839) (end 126.946398 93.926398) (width 0.2) (layer "F.Cu") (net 13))
 (segment (start 123.168559 93.947839) (end 126.924957 93.947839) (width 0.2) (layer "F.Cu") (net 13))
 (segment (start 126.924957 121.887839) (end 126.946398 121.866398) (width 0.2) (layer "F.Cu") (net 22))
 (segment (start 123.168559 121.887839) (end 126.924957 121.887839) (width 0.2) (layer "F.Cu") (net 22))
 (segment (start 123.168559 124.427839) (end 126.924957 124.427839) (width 0.2) (layer "F.Cu") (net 23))
 (segment (start 126.924957 124.427839) (end 126.946398 124.406398) (width 0.2) (layer "F.Cu") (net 23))
 (segment (start 123.168559 81.247839) (end 126.924957 81.247839) (width 0.2) (layer "F.Cu") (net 9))
 (segment (start 126.924957 81.247839) (end 126.946398 81.226398) (width 0.2) (layer "F.Cu") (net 9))
 (segment (start 123.168559 116.807839) (end 126.924957 116.807839) (width 0.2) (layer "F.Cu") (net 20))
 (segment (start 126.924957 116.807839) (end 126.946398 116.786398) (width 0.2) (layer "F.Cu") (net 20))
 (segment (start 126.924957 96.487839) (end 126.946398 96.466398) (width 0.2) (layer "F.Cu") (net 14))
 (segment (start 123.168559 96.487839) (end 126.924957 96.487839) (width 0.2) (layer "F.Cu") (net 14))
 (segment (start 123.168559 104.107839) (end 126.924957 104.107839) (width 0.2) (layer "F.Cu") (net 17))
 (segment (start 126.924957 104.107839) (end 126.946398 104.086398) (width 0.2) (layer "F.Cu") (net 17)))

